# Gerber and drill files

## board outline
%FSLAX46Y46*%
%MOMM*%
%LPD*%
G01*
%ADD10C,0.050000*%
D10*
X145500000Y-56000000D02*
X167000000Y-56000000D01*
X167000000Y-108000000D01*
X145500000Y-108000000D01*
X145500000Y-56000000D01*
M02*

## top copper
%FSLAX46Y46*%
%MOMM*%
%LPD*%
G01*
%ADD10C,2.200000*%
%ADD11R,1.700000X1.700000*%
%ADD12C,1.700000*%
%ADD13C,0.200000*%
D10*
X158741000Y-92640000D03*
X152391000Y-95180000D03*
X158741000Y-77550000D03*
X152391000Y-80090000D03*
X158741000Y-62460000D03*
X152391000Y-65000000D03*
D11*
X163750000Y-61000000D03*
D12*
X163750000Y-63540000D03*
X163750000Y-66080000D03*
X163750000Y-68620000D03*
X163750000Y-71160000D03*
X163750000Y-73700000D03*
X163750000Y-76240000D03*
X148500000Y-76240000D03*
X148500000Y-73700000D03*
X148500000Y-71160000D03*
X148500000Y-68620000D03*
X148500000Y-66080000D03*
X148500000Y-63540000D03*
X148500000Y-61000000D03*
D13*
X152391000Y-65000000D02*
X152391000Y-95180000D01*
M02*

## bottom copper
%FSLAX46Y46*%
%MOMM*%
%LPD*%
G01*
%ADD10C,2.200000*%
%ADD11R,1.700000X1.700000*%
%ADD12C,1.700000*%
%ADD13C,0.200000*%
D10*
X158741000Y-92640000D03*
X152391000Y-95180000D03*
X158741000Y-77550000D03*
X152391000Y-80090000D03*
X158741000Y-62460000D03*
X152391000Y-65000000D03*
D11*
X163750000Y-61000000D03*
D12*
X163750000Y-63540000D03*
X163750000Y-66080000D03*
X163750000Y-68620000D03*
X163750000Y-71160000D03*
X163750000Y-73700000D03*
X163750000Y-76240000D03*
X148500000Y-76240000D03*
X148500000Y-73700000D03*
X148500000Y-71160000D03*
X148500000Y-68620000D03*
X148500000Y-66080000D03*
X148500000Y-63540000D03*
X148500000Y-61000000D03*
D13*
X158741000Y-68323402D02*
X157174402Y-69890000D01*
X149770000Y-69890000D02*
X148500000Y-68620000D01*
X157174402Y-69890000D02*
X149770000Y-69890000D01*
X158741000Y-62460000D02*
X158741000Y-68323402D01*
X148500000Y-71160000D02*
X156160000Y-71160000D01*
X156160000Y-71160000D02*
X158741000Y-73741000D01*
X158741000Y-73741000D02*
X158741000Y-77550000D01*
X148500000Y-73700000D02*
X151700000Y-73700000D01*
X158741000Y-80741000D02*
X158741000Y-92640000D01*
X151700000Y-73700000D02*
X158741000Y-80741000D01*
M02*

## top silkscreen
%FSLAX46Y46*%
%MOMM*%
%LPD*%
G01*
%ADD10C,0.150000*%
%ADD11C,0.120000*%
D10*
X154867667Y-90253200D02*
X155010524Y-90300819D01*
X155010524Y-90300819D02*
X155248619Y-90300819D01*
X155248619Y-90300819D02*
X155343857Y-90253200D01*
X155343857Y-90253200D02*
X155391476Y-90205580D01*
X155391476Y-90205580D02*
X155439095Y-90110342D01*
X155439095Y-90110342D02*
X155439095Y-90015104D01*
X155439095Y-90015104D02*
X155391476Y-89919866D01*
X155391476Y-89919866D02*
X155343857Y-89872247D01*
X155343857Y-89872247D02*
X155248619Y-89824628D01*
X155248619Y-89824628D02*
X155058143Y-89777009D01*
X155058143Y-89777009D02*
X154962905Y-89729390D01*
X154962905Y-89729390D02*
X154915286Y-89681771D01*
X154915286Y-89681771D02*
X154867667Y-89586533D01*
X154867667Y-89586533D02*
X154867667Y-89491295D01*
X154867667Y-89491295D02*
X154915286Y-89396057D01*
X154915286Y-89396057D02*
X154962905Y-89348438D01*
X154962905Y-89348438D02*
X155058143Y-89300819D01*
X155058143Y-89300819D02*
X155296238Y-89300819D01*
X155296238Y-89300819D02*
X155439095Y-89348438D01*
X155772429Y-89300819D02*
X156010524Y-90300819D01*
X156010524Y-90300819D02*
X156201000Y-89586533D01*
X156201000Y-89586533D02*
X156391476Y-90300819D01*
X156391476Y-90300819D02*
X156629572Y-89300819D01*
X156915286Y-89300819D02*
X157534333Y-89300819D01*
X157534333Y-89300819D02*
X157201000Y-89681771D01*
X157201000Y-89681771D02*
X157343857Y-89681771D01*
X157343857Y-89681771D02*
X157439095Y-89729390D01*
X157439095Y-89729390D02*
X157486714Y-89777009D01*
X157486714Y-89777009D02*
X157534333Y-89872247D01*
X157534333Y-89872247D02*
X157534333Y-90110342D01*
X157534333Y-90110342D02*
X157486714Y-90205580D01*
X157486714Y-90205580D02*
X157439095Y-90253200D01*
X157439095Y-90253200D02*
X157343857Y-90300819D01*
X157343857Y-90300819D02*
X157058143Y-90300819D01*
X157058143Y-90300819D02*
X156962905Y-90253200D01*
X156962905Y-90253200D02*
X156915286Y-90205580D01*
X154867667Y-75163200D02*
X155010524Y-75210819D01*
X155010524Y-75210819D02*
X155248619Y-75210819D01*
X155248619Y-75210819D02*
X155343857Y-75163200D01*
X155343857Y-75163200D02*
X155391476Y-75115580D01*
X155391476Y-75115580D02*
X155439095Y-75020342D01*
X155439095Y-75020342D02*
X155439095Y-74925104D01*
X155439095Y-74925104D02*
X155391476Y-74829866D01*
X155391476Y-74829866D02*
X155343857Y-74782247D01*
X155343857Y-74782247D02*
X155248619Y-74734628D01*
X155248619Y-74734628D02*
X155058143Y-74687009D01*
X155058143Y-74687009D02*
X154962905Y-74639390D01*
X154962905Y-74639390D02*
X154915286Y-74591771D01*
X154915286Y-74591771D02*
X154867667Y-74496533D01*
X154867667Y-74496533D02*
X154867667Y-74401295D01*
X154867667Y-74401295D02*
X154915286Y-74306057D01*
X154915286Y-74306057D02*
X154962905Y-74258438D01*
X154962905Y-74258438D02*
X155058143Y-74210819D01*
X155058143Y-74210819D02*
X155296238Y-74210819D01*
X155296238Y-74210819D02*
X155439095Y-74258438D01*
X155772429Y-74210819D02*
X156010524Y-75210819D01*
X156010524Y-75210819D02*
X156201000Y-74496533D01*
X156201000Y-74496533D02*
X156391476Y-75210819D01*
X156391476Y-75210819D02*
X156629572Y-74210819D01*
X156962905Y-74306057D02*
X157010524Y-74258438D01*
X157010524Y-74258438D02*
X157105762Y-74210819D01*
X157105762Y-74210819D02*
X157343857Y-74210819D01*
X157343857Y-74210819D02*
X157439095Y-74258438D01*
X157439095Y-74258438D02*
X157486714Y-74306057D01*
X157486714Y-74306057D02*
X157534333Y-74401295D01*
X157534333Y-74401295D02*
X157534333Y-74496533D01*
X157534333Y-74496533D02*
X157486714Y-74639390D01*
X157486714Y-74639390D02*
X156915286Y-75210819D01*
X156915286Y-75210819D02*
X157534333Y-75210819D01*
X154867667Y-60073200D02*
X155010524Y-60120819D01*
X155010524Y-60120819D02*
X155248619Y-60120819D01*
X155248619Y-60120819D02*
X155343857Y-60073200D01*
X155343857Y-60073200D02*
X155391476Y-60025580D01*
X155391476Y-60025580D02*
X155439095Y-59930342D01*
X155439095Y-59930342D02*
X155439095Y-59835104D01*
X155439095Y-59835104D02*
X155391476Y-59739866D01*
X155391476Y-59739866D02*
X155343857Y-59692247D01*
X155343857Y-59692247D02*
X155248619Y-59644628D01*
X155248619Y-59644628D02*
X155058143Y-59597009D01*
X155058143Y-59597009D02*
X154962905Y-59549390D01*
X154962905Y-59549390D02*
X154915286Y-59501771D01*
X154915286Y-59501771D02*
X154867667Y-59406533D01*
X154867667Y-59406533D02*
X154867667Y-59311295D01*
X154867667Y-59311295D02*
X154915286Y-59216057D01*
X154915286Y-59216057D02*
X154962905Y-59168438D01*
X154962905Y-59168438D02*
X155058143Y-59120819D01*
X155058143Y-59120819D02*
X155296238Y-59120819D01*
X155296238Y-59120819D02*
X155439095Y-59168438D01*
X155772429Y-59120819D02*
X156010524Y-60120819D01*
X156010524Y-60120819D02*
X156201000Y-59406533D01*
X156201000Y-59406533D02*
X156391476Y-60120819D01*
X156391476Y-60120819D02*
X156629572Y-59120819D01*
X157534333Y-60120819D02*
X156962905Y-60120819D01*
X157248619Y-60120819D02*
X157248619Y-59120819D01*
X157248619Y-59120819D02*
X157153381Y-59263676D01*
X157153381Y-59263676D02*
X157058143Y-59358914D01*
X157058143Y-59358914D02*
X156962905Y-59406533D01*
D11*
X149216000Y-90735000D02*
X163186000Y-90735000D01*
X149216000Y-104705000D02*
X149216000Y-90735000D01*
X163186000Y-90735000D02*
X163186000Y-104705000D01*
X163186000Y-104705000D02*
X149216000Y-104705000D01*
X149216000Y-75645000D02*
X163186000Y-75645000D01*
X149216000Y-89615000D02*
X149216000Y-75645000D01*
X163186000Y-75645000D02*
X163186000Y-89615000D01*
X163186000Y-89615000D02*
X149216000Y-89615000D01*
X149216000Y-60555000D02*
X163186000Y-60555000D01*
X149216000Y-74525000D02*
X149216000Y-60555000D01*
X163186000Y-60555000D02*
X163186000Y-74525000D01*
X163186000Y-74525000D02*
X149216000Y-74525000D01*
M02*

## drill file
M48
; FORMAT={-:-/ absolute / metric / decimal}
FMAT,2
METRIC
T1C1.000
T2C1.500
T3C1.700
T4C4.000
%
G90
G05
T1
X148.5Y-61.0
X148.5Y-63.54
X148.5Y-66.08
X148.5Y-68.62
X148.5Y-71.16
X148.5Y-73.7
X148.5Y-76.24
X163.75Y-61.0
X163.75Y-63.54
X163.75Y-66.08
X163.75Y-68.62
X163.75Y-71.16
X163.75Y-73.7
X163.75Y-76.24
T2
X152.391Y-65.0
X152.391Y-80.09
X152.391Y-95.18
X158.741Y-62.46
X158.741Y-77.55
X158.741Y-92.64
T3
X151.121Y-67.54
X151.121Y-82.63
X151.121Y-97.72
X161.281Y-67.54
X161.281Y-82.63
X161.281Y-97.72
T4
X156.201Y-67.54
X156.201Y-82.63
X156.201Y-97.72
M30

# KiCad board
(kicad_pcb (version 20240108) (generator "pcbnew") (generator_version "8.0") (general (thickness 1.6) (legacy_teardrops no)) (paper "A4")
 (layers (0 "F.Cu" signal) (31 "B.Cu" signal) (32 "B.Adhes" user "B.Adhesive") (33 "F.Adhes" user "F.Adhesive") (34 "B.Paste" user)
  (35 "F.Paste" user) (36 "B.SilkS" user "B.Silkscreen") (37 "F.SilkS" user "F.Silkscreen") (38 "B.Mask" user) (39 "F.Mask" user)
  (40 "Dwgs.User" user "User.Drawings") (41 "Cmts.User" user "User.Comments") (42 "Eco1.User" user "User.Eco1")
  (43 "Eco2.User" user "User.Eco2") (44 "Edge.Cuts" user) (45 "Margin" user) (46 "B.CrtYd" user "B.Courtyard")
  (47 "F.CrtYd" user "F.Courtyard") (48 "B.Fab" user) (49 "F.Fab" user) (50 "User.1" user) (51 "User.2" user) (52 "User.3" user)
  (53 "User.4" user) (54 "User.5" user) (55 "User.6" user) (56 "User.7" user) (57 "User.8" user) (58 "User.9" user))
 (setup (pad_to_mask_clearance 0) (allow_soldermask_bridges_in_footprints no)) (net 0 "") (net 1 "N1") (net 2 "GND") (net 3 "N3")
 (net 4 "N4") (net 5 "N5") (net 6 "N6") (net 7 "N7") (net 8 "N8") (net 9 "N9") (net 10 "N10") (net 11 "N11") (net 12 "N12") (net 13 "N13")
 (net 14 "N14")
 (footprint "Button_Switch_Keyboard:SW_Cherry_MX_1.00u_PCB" (layer "F.Cu") (at 158.741 92.64)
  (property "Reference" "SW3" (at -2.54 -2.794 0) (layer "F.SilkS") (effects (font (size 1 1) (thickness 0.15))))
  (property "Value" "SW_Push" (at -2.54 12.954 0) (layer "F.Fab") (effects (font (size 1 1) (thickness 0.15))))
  (fp_line (start -9.525 -1.905) (end 4.445 -1.905) (stroke (width 0.12) (type solid)) (layer "F.SilkS"))
  (fp_line (start -9.525 12.065) (end -9.525 -1.905) (stroke (width 0.12) (type solid)) (layer "F.SilkS"))
  (fp_line (start 4.445 -1.905) (end 4.445 12.065) (stroke (width 0.12) (type solid)) (layer "F.SilkS"))
  (fp_line (start 4.445 12.065) (end -9.525 12.065) (stroke (width 0.12) (type solid)) (layer "F.SilkS"))
  (pad "" np_thru_hole circle (at -7.62 5.08) (size 1.7 1.7) (drill 1.7) (layers "*.Cu" "*.Mask"))
  (pad "" np_thru_hole circle (at -2.54 5.08) (size 4 4) (drill 4) (layers "*.Cu" "*.Mask"))
  (pad "" np_thru_hole circle (at 2.54 5.08) (size 1.7 1.7) (drill 1.7) (layers "*.Cu" "*.Mask"))
  (pad "1" thru_hole circle (at 0 0) (size 2.2 2.2) (drill 1.5) (layers "*.Cu" "*.Mask") (remove_unused_layers no) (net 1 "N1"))
  (pad "2" thru_hole circle (at -6.35 2.54) (size 2.2 2.2) (drill 1.5) (layers "*.Cu" "*.Mask") (remove_unused_layers no) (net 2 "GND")))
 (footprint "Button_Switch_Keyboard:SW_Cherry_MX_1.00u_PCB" (layer "F.Cu") (at 158.741 77.55)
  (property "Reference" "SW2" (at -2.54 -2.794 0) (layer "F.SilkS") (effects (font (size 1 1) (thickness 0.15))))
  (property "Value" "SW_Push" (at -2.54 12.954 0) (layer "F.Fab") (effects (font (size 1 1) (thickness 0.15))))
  (fp_line (start -9.525 -1.905) (end 4.445 -1.905) (stroke (width 0.12) (type solid)) (layer "F.SilkS"))
  (fp_line (start -9.525 12.065) (end -9.525 -1.905) (stroke (width 0.12) (type solid)) (layer "F.SilkS"))
  (fp_line (start 4.445 -1.905) (end 4.445 12.065) (stroke (width 0.12) (type solid)) (layer "F.SilkS"))
  (fp_line (start 4.445 12.065) (end -9.525 12.065) (stroke (width 0.12) (type solid)) (layer "F.SilkS"))
  (pad "" np_thru_hole circle (at -7.62 5.08) (size 1.7 1.7) (drill 1.7) (layers "*.Cu" "*.Mask"))
  (pad "" np_thru_hole circle (at -2.54 5.08) (size 4 4) (drill 4) (layers "*.Cu" "*.Mask"))
  (pad "" np_thru_hole circle (at 2.54 5.08) (size 1.7 1.7) (drill 1.7) (layers "*.Cu" "*.Mask"))
  (pad "1" thru_hole circle (at 0 0) (size 2.2 2.2) (drill 1.5) (layers "*.Cu" "*.Mask") (remove_unused_layers no) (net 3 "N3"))
  (pad "2" thru_hole circle (at -6.35 2.54) (size 2.2 2.2) (drill 1.5) (layers "*.Cu" "*.Mask") (remove_unused_layers no) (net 2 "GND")))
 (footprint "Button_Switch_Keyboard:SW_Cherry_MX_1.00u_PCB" (layer "F.Cu") (at 158.741 62.46)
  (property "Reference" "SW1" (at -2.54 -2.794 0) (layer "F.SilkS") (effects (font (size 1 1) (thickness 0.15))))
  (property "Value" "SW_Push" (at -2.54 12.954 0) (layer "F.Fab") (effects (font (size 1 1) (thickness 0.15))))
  (fp_line (start -9.525 -1.905) (end 4.445 -1.905) (stroke (width 0.12) (type solid)) (layer "F.SilkS"))
  (fp_line (start -9.525 12.065) (end -9.525 -1.905) (stroke (width 0.12) (type solid)) (layer "F.SilkS"))
  (fp_line (start 4.445 -1.905) (end 4.445 12.065) (stroke (width 0.12) (type solid)) (layer "F.SilkS"))
  (fp_line (start 4.445 12.065) (end -9.525 12.065) (stroke (width 0.12) (type solid)) (layer "F.SilkS"))
  (pad "" np_thru_hole circle (at -7.62 5.08) (size 1.7 1.7) (drill 1.7) (layers "*.Cu" "*.Mask"))
  (pad "" np_thru_hole circle (at -2.54 5.08) (size 4 4) (drill 4) (layers "*.Cu" "*.Mask"))
  (pad "" np_thru_hole circle (at 2.54 5.08) (size 1.7 1.7) (drill 1.7) (layers "*.Cu" "*.Mask"))
  (pad "1" thru_hole circle (at 0 0) (size 2.2 2.2) (drill 1.5) (layers "*.Cu" "*.Mask") (remove_unused_layers no) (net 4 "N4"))
  (pad "2" thru_hole circle (at -6.35 2.54) (size 2.2 2.2) (drill 1.5) (layers "*.Cu" "*.Mask") (remove_unused_layers no) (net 2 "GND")))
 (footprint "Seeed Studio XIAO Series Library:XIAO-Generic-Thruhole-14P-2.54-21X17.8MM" (layer "B.Cu") (at 156.125 68.62 180)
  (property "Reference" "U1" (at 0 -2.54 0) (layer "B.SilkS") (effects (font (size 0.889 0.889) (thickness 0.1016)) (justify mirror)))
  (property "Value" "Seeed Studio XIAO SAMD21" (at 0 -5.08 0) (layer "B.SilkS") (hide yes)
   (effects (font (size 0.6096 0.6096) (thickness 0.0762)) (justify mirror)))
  (pad "1" thru_hole rect (at -7.625 7.62 180) (size 1.7 1.7) (drill 1) (layers "*.Cu" "*.Mask") (remove_unused_layers no) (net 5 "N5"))
  (pad "2" thru_hole circle (at -7.625 5.08 180) (size 1.7 1.7) (drill 1) (layers "*.Cu" "*.Mask") (remove_unused_layers no) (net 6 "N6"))
  (pad "3" thru_hole circle (at -7.625 2.54 180) (size 1.7 1.7) (drill 1) (layers "*.Cu" "*.Mask") (remove_unused_layers no) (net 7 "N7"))
  (pad "4" thru_hole circle (at -7.625 0 180) (size 1.7 1.7) (drill 1) (layers "*.Cu" "*.Mask") (remove_unused_layers no) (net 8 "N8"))
  (pad "5" thru_hole circle (at -7.625 -2.54 180) (size 1.7 1.7) (drill 1) (layers "*.Cu" "*.Mask") (remove_unused_layers no) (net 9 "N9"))
  (pad "6" thru_hole circle (at -7.625 -5.08) (size 1.7 1.7) (drill 1) (layers "*.Cu" "*.Mask") (remove_unused_layers no) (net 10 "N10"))
  (pad "7" thru_hole circle (at -7.625 -7.62 180) (size 1.7 1.7) (drill 1) (layers "*.Cu" "*.Mask") (remove_unused_layers no) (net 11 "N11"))
  (pad "8" thru_hole circle (at 7.625 -7.62 180) (size 1.7 1.7) (drill 1) (layers "*.Cu" "*.Mask") (remove_unused_layers no) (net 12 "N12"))
  (pad "9" thru_hole circle (at 7.625 -5.08 180) (size 1.7 1.7) (drill 1) (layers "*.Cu" "*.Mask") (remove_unused_layers no) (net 1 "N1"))
  (pad "10" thru_hole circle (at 7.625 -2.54 180) (size 1.7 1.7) (drill 1) (layers "*.Cu" "*.Mask") (remove_unused_layers no) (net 3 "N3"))
  (pad "11" thru_hole circle (at 7.625 0 180) (size 1.7 1.7) (drill 1) (layers "*.Cu" "*.Mask") (remove_unused_layers no) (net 4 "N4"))
  (pad "12" thru_hole circle (at 7.625 2.54 180) (size 1.7 1.7) (drill 1) (layers "*.Cu" "*.Mask") (remove_unused_layers no) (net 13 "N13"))
  (pad "13" thru_hole circle (at 7.625 5.08 180) (size 1.7 1.7) (drill 1) (layers "*.Cu" "*.Mask") (remove_unused_layers no) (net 2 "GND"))
  (pad "14" thru_hole circle (at 7.625 7.62 180) (size 1.7 1.7) (drill 1) (layers "*.Cu" "*.Mask") (remove_unused_layers no) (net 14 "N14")))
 (gr_rect (start 145.5 56) (end 167 108) (stroke (width 0.05) (type default)) (fill none) (layer "Edge.Cuts"))
 (segment (start 152.391 65) (end 152.391 95.18) (width 0.2) (layer "F.Cu") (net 2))
 (segment (start 158.741 68.323402) (end 157.174402 69.89) (width 0.2) (layer "B.Cu") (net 4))
 (segment (start 149.77 69.89) (end 148.5 68.62) (width 0.2) (layer "B.Cu") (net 4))
 (segment (start 157.174402 69.89) (end 149.77 69.89) (width 0.2) (layer "B.Cu") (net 4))
 (segment (start 158.741 62.46) (end 158.741 68.323402) (width 0.2) (layer "B.Cu") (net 4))
 (segment (start 148.5 71.16) (end 156.16 71.16) (width 0.2) (layer "B.Cu") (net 3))
 (segment (start 156.16 71.16) (end 158.741 73.741) (width 0.2) (layer "B.Cu") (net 3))
 (segment (start 158.741 73.741) (end 158.741 77.55) (width 0.2) (layer "B.Cu") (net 3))
 (segment (start 148.5 73.7) (end 151.7 73.7) (width 0.2) (layer "B.Cu") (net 1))
 (segment (start 158.741 80.741) (end 158.741 92.64) (width 0.2) (layer "B.Cu") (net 1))
 (segment (start 151.7 73.7) (end 158.741 80.741) (width 0.2) (layer "B.Cu") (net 1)))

